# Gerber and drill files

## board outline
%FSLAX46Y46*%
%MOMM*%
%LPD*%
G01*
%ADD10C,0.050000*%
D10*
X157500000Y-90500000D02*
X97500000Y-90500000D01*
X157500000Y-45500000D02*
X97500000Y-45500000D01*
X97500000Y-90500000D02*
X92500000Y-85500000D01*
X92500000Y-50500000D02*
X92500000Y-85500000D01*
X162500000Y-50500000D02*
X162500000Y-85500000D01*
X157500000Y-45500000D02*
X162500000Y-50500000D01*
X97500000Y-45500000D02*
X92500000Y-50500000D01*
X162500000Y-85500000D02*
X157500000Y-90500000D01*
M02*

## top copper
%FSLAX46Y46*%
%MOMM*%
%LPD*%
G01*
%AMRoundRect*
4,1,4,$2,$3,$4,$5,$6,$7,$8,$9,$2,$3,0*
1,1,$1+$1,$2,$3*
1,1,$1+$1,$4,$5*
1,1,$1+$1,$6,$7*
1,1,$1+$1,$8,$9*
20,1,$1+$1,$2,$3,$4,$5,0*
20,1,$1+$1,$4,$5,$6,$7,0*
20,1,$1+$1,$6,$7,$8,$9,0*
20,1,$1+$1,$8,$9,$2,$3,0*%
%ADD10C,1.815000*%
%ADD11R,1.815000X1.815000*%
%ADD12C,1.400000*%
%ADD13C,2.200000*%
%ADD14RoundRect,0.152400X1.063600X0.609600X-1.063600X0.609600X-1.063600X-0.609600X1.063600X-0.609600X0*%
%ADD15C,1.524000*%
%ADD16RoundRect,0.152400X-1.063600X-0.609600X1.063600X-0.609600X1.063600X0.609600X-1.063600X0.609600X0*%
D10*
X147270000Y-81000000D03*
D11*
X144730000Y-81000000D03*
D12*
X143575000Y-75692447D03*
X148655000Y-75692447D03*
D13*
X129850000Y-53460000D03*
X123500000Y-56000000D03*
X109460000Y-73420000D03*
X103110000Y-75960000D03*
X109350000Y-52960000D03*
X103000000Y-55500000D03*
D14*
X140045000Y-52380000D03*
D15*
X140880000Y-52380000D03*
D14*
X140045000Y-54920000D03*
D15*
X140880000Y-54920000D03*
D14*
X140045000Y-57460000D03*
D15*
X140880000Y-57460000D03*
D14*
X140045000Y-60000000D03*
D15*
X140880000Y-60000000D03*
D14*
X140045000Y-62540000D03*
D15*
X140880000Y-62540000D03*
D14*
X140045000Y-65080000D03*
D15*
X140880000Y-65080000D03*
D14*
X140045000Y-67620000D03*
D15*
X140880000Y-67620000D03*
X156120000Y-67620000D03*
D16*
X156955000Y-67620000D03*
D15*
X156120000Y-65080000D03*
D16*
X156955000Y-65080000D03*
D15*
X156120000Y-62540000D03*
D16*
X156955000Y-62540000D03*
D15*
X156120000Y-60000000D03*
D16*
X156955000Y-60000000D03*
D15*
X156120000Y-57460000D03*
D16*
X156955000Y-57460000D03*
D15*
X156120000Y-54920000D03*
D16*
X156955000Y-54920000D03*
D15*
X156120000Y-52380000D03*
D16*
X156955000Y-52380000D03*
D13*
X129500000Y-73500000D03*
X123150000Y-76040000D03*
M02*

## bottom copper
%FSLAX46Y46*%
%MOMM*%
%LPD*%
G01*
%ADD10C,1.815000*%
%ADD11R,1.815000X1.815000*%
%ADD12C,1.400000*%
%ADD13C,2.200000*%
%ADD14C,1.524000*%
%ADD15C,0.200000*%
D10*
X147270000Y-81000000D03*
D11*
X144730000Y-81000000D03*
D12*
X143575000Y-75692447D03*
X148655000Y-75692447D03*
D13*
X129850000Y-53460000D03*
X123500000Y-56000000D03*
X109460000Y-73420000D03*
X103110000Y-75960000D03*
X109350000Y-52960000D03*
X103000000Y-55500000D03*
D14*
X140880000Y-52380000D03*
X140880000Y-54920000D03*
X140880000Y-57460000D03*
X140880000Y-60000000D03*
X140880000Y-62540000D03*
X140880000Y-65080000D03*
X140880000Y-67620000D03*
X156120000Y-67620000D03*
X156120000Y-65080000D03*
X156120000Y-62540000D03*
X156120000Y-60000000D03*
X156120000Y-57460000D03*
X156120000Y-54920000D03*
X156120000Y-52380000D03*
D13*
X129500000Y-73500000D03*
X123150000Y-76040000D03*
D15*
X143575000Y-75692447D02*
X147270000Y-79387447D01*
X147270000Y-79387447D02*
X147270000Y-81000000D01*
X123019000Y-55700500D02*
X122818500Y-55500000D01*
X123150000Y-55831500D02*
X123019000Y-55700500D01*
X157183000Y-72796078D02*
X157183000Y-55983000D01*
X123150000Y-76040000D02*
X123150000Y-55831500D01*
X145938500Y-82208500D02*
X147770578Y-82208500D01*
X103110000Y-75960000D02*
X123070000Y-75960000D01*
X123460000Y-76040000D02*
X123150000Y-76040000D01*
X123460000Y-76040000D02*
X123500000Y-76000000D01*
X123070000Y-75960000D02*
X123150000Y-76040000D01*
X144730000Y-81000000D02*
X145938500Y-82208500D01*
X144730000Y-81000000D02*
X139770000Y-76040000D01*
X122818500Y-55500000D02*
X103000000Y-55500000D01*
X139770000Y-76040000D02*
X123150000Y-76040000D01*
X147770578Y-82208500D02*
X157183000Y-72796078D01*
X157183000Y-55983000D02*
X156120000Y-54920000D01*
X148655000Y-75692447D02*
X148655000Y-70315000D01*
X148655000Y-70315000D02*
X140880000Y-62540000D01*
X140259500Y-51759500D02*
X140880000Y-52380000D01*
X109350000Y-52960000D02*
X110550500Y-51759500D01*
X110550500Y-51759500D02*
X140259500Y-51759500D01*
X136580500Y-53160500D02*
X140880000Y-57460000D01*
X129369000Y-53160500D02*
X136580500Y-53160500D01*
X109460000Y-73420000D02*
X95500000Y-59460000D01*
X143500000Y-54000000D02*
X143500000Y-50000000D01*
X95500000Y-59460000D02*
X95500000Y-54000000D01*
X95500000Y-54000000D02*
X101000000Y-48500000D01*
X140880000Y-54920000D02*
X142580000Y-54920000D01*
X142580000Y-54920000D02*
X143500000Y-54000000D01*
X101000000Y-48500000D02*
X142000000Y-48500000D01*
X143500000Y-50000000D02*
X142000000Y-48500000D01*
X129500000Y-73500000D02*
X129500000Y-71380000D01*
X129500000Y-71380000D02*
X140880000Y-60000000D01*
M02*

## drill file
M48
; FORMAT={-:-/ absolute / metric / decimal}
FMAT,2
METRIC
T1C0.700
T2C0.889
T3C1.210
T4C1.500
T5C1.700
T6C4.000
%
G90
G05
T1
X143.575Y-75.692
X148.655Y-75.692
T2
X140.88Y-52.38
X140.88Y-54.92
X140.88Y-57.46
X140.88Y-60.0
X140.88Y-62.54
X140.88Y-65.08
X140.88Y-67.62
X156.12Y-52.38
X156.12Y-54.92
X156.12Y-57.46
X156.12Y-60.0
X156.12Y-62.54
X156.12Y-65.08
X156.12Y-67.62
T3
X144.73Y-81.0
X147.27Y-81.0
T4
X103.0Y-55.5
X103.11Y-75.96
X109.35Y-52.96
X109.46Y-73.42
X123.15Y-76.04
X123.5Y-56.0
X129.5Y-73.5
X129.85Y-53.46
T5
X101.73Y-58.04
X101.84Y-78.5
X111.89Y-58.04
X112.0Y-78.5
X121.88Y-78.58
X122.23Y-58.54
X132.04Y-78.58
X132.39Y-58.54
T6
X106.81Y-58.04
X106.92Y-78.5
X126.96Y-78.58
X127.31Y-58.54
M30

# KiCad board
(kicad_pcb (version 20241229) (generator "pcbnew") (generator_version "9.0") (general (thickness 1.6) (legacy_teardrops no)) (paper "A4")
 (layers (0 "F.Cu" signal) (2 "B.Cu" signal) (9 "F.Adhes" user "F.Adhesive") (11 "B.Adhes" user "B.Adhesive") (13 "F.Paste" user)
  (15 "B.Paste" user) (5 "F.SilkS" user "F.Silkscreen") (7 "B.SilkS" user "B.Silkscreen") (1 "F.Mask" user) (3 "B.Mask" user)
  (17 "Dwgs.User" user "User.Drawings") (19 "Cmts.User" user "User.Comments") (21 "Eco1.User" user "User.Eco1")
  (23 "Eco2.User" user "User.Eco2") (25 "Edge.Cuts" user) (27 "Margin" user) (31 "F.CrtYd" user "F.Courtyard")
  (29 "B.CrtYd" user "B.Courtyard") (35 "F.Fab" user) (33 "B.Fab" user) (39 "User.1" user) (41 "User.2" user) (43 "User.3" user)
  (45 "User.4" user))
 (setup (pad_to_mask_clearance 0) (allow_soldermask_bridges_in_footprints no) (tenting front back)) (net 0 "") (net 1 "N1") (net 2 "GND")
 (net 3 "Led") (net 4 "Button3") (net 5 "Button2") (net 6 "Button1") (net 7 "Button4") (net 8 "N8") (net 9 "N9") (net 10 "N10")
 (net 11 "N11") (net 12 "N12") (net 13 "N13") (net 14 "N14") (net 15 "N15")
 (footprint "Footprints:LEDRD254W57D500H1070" (layer "F.Cu") (at 146 81)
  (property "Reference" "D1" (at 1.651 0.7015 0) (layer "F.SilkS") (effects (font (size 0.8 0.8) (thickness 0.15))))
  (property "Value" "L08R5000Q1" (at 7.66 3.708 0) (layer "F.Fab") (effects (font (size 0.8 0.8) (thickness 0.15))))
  (pad "A" thru_hole circle (at 1.27 0) (size 1.815 1.815) (drill 1.21) (layers "*.Cu" "*.Mask") (remove_unused_layers no) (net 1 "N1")
   (solder_mask_margin 0.102))
  (pad "C" thru_hole rect (at -1.27 0) (size 1.815 1.815) (drill 1.21) (layers "*.Cu" "*.Mask") (remove_unused_layers no) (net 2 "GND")
   (solder_mask_margin 0.102)))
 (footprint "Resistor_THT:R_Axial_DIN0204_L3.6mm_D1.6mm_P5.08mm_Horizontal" (layer "F.Cu") (at 143.575 75.692447)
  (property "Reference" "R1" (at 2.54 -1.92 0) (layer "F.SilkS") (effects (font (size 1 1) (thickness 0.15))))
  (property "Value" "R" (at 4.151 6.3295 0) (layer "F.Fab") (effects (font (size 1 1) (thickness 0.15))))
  (pad "1" thru_hole circle (at 0 0) (size 1.4 1.4) (drill 0.7) (layers "*.Cu" "*.Mask") (remove_unused_layers no) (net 1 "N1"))
  (pad "2" thru_hole circle (at 5.08 0) (size 1.4 1.4) (drill 0.7) (layers "*.Cu" "*.Mask") (remove_unused_layers no) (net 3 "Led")))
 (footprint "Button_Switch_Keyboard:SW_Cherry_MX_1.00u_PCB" (layer "F.Cu") (at 129.85 53.46)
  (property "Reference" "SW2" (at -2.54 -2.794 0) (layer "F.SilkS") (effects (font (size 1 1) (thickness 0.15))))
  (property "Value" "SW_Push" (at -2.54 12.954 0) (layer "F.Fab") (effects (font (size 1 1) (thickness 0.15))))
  (pad "" np_thru_hole circle (at -7.62 5.08) (size 1.7 1.7) (drill 1.7) (layers "*.Cu" "*.Mask"))
  (pad "" np_thru_hole circle (at -2.54 5.08) (size 4 4) (drill 4) (layers "*.Cu" "*.Mask"))
  (pad "" np_thru_hole circle (at 2.54 5.08) (size 1.7 1.7) (drill 1.7) (layers "*.Cu" "*.Mask"))
  (pad "1" thru_hole circle (at 0 0) (size 2.2 2.2) (drill 1.5) (layers "*.Cu" "*.Mask") (remove_unused_layers no) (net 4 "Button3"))
  (pad "2" thru_hole circle (at -6.35 2.54) (size 2.2 2.2) (drill 1.5) (layers "*.Cu" "*.Mask") (remove_unused_layers no) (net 2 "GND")))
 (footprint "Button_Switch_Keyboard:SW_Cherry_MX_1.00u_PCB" (layer "F.Cu") (at 109.46 73.42)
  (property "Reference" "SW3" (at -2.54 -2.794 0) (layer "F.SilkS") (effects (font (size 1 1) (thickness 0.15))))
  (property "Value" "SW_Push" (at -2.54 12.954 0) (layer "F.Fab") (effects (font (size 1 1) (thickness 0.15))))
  (pad "" np_thru_hole circle (at -7.62 5.08) (size 1.7 1.7) (drill 1.7) (layers "*.Cu" "*.Mask"))
  (pad "" np_thru_hole circle (at -2.54 5.08) (size 4 4) (drill 4) (layers "*.Cu" "*.Mask"))
  (pad "" np_thru_hole circle (at 2.54 5.08) (size 1.7 1.7) (drill 1.7) (layers "*.Cu" "*.Mask"))
  (pad "1" thru_hole circle (at 0 0) (size 2.2 2.2) (drill 1.5) (layers "*.Cu" "*.Mask") (remove_unused_layers no) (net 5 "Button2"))
  (pad "2" thru_hole circle (at -6.35 2.54) (size 2.2 2.2) (drill 1.5) (layers "*.Cu" "*.Mask") (remove_unused_layers no) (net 2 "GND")))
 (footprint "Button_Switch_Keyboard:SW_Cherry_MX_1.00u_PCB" (layer "F.Cu") (at 109.35 52.96)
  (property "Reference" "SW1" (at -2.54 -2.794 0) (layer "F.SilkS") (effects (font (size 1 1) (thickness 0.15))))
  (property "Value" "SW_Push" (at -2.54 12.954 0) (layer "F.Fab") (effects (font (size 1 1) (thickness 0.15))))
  (pad "" np_thru_hole circle (at -7.62 5.08) (size 1.7 1.7) (drill 1.7) (layers "*.Cu" "*.Mask"))
  (pad "" np_thru_hole circle (at -2.54 5.08) (size 4 4) (drill 4) (layers "*.Cu" "*.Mask"))
  (pad "" np_thru_hole circle (at 2.54 5.08) (size 1.7 1.7) (drill 1.7) (layers "*.Cu" "*.Mask"))
  (pad "1" thru_hole circle (at 0 0) (size 2.2 2.2) (drill 1.5) (layers "*.Cu" "*.Mask") (remove_unused_layers no) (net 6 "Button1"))
  (pad "2" thru_hole circle (at -6.35 2.54) (size 2.2 2.2) (drill 1.5) (layers "*.Cu" "*.Mask") (remove_unused_layers no) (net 2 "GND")))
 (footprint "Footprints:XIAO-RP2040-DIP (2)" (layer "F.Cu") (at 148.5 60)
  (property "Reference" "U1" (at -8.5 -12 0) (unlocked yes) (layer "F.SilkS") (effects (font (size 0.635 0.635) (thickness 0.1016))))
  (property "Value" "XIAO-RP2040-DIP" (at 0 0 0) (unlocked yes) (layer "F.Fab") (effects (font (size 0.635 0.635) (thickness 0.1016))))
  (pad "1" smd roundrect (at -8.455 -7.62 180) (size 2.432 1.524) (layers "F.Cu" "F.Mask") (roundrect_rratio 0.1) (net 6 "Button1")
   (thermal_bridge_angle 45))
  (pad "1" thru_hole circle (at -7.62 -7.62 180) (size 1.524 1.524) (drill 0.889) (layers "*.Cu" "*.Mask") (remove_unused_layers no)
   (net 6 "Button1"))
  (pad "2" smd roundrect (at -8.455 -5.08 180) (size 2.432 1.524) (layers "F.Cu" "F.Mask") (roundrect_rratio 0.1) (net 5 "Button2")
   (thermal_bridge_angle 45))
  (pad "2" thru_hole circle (at -7.62 -5.08 180) (size 1.524 1.524) (drill 0.889) (layers "*.Cu" "*.Mask") (remove_unused_layers no)
   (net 5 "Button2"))
  (pad "3" smd roundrect (at -8.455 -2.54 180) (size 2.432 1.524) (layers "F.Cu" "F.Mask") (roundrect_rratio 0.1) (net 4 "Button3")
   (thermal_bridge_angle 45))
  (pad "3" thru_hole circle (at -7.62 -2.54 180) (size 1.524 1.524) (drill 0.889) (layers "*.Cu" "*.Mask") (remove_unused_layers no)
   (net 4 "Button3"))
  (pad "4" smd roundrect (at -8.455 0 180) (size 2.432 1.524) (layers "F.Cu" "F.Mask") (roundrect_rratio 0.1) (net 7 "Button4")
   (thermal_bridge_angle 45))
  (pad "4" thru_hole circle (at -7.62 0 180) (size 1.524 1.524) (drill 0.889) (layers "*.Cu" "*.Mask") (remove_unused_layers no)
   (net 7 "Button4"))
  (pad "5" smd roundrect (at -8.455 2.54 180) (size 2.432 1.524) (layers "F.Cu" "F.Mask") (roundrect_rratio 0.1) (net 3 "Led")
   (thermal_bridge_angle 45))
  (pad "5" thru_hole circle (at -7.62 2.54 180) (size 1.524 1.524) (drill 0.889) (layers "*.Cu" "*.Mask") (remove_unused_layers no)
   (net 3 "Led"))
  (pad "6" smd roundrect (at -8.455 5.08 180) (size 2.432 1.524) (layers "F.Cu" "F.Mask") (roundrect_rratio 0.1) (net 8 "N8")
   (thermal_bridge_angle 45))
  (pad "6" thru_hole circle (at -7.62 5.08 180) (size 1.524 1.524) (drill 0.889) (layers "*.Cu" "*.Mask") (remove_unused_layers no)
   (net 8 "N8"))
  (pad "7" smd roundrect (at -8.455 7.62 180) (size 2.432 1.524) (layers "F.Cu" "F.Mask") (roundrect_rratio 0.1) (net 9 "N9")
   (thermal_bridge_angle 45))
  (pad "7" thru_hole circle (at -7.62 7.62 180) (size 1.524 1.524) (drill 0.889) (layers "*.Cu" "*.Mask") (remove_unused_layers no)
   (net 9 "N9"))
  (pad "8" thru_hole circle (at 7.62 7.62) (size 1.524 1.524) (drill 0.889) (layers "*.Cu" "*.Mask") (remove_unused_layers no)
   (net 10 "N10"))
  (pad "8" smd roundrect (at 8.455 7.62) (size 2.432 1.524) (layers "F.Cu" "F.Mask") (roundrect_rratio 0.1) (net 10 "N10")
   (thermal_bridge_angle 45))
  (pad "9" thru_hole circle (at 7.62 5.08) (size 1.524 1.524) (drill 0.889) (layers "*.Cu" "*.Mask") (remove_unused_layers no)
   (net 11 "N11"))
  (pad "9" smd roundrect (at 8.455 5.08) (size 2.432 1.524) (layers "F.Cu" "F.Mask") (roundrect_rratio 0.1) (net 11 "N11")
   (thermal_bridge_angle 45))
  (pad "10" thru_hole circle (at 7.62 2.54) (size 1.524 1.524) (drill 0.889) (layers "*.Cu" "*.Mask") (remove_unused_layers no)
   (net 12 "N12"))
  (pad "10" smd roundrect (at 8.455 2.54) (size 2.432 1.524) (layers "F.Cu" "F.Mask") (roundrect_rratio 0.1) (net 12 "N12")
   (thermal_bridge_angle 45))
  (pad "11" thru_hole circle (at 7.62 0) (size 1.524 1.524) (drill 0.889) (layers "*.Cu" "*.Mask") (remove_unused_layers no) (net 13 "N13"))
  (pad "11" smd roundrect (at 8.455 0) (size 2.432 1.524) (layers "F.Cu" "F.Mask") (roundrect_rratio 0.1) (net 13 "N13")
   (thermal_bridge_angle 45))
  (pad "12" thru_hole circle (at 7.62 -2.54) (size 1.524 1.524) (drill 0.889) (layers "*.Cu" "*.Mask") (remove_unused_layers no)
   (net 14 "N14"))
  (pad "12" smd roundrect (at 8.455 -2.54) (size 2.432 1.524) (layers "F.Cu" "F.Mask") (roundrect_rratio 0.1) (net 14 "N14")
   (thermal_bridge_angle 45))
  (pad "13" thru_hole circle (at 7.62 -5.08) (size 1.524 1.524) (drill 0.889) (layers "*.Cu" "*.Mask") (remove_unused_layers no)
   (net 2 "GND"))
  (pad "13" smd roundrect (at 8.455 -5.08) (size 2.432 1.524) (layers "F.Cu" "F.Mask") (roundrect_rratio 0.1) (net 2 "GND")
   (thermal_bridge_angle 45))
  (pad "14" thru_hole circle (at 7.62 -7.62) (size 1.524 1.524) (drill 0.889) (layers "*.Cu" "*.Mask") (remove_unused_layers no)
   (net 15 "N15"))
  (pad "14" smd roundrect (at 8.455 -7.62) (size 2.432 1.524) (layers "F.Cu" "F.Mask") (roundrect_rratio 0.1) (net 15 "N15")
   (thermal_bridge_angle 45)))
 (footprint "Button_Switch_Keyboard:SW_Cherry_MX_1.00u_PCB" (layer "F.Cu") (at 129.5 73.5)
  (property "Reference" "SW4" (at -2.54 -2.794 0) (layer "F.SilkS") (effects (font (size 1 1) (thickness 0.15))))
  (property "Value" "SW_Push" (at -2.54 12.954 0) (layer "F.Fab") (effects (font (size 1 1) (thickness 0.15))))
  (pad "" np_thru_hole circle (at -7.62 5.08) (size 1.7 1.7) (drill 1.7) (layers "*.Cu" "*.Mask"))
  (pad "" np_thru_hole circle (at -2.54 5.08) (size 4 4) (drill 4) (layers "*.Cu" "*.Mask"))
  (pad "" np_thru_hole circle (at 2.54 5.08) (size 1.7 1.7) (drill 1.7) (layers "*.Cu" "*.Mask"))
  (pad "1" thru_hole circle (at 0 0) (size 2.2 2.2) (drill 1.5) (layers "*.Cu" "*.Mask") (remove_unused_layers no) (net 7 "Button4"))
  (pad "2" thru_hole circle (at -6.35 2.54) (size 2.2 2.2) (drill 1.5) (layers "*.Cu" "*.Mask") (remove_unused_layers no) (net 2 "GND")))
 (gr_line (start 157.5 90.5) (end 97.5 90.5) (stroke (width 0.05) (type default)) (layer "Edge.Cuts"))
 (gr_line (start 157.5 45.5) (end 97.5 45.5) (stroke (width 0.05) (type default)) (layer "Edge.Cuts"))
 (gr_line (start 97.5 90.5) (end 92.5 85.5) (stroke (width 0.05) (type default)) (layer "Edge.Cuts"))
 (gr_line (start 92.5 50.5) (end 92.5 85.5) (stroke (width 0.05) (type default)) (layer "Edge.Cuts"))
 (gr_line (start 162.5 50.5) (end 162.5 85.5) (stroke (width 0.05) (type default)) (layer "Edge.Cuts"))
 (gr_line (start 157.5 45.5) (end 162.5 50.5) (stroke (width 0.05) (type default)) (layer "Edge.Cuts"))
 (gr_line (start 97.5 45.5) (end 92.5 50.5) (stroke (width 0.05) (type default)) (layer "Edge.Cuts"))
 (gr_line (start 162.5 85.5) (end 157.5 90.5) (stroke (width 0.05) (type default)) (layer "Edge.Cuts"))
 (segment (start 143.575 75.692447) (end 147.27 79.387447) (width 0.2) (layer "B.Cu") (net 1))
 (segment (start 147.27 79.387447) (end 147.27 81) (width 0.2) (layer "B.Cu") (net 1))
 (segment (start 123.019 55.7005) (end 122.8185 55.5) (width 0.2) (layer "B.Cu") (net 2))
 (segment (start 123.15 55.8315) (end 123.019 55.7005) (width 0.2) (layer "B.Cu") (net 2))
 (segment (start 157.183 72.796078) (end 157.183 55.983) (width 0.2) (layer "B.Cu") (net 2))
 (segment (start 123.15 76.04) (end 123.15 55.8315) (width 0.2) (layer "B.Cu") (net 2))
 (segment (start 145.9385 82.2085) (end 147.770578 82.2085) (width 0.2) (layer "B.Cu") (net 2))
 (segment (start 103.11 75.96) (end 123.07 75.96) (width 0.2) (layer "B.Cu") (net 2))
 (segment (start 123.46 76.04) (end 123.15 76.04) (width 0.2) (layer "B.Cu") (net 2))
 (segment (start 123.46 76.04) (end 123.5 76) (width 0.2) (layer "B.Cu") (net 2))
 (segment (start 123.07 75.96) (end 123.15 76.04) (width 0.2) (layer "B.Cu") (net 2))
 (segment (start 144.73 81) (end 145.9385 82.2085) (width 0.2) (layer "B.Cu") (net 2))
 (segment (start 144.73 81) (end 139.77 76.04) (width 0.2) (layer "B.Cu") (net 2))
 (segment (start 122.8185 55.5) (end 103 55.5) (width 0.2) (layer "B.Cu") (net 2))
 (segment (start 139.77 76.04) (end 123.15 76.04) (width 0.2) (layer "B.Cu") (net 2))
 (segment (start 147.770578 82.2085) (end 157.183 72.796078) (width 0.2) (layer "B.Cu") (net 2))
 (segment (start 157.183 55.983) (end 156.12 54.92) (width 0.2) (layer "B.Cu") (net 2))
 (segment (start 148.655 75.692447) (end 148.655 70.315) (width 0.2) (layer "B.Cu") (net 3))
 (segment (start 148.655 70.315) (end 140.88 62.54) (width 0.2) (layer "B.Cu") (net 3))
 (segment (start 140.2595 51.7595) (end 140.88 52.38) (width 0.2) (layer "B.Cu") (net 6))
 (segment (start 109.35 52.96) (end 110.5505 51.7595) (width 0.2) (layer "B.Cu") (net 6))
 (segment (start 110.5505 51.7595) (end 140.2595 51.7595) (width 0.2) (layer "B.Cu") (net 6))
 (segment (start 136.5805 53.1605) (end 140.88 57.46) (width 0.2) (layer "B.Cu") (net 4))
 (segment (start 129.369 53.1605) (end 136.5805 53.1605) (width 0.2) (layer "B.Cu") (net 4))
 (segment (start 109.46 73.42) (end 95.5 59.46) (width 0.2) (layer "B.Cu") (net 5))
 (segment (start 143.5 54) (end 143.5 50) (width 0.2) (layer "B.Cu") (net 5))
 (segment (start 95.5 59.46) (end 95.5 54) (width 0.2) (layer "B.Cu") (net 5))
 (segment (start 95.5 54) (end 101 48.5) (width 0.2) (layer "B.Cu") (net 5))
 (segment (start 140.88 54.92) (end 142.58 54.92) (width 0.2) (layer "B.Cu") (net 5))
 (segment (start 142.58 54.92) (end 143.5 54) (width 0.2) (layer "B.Cu") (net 5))
 (segment (start 101 48.5) (end 142 48.5) (width 0.2) (layer "B.Cu") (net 5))
 (segment (start 143.5 50) (end 142 48.5) (width 0.2) (layer "B.Cu") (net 5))
 (segment (start 129.5 73.5) (end 129.5 71.38) (width 0.2) (layer "B.Cu") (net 7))
 (segment (start 129.5 71.38) (end 140.88 60) (width 0.2) (layer "B.Cu") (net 7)))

